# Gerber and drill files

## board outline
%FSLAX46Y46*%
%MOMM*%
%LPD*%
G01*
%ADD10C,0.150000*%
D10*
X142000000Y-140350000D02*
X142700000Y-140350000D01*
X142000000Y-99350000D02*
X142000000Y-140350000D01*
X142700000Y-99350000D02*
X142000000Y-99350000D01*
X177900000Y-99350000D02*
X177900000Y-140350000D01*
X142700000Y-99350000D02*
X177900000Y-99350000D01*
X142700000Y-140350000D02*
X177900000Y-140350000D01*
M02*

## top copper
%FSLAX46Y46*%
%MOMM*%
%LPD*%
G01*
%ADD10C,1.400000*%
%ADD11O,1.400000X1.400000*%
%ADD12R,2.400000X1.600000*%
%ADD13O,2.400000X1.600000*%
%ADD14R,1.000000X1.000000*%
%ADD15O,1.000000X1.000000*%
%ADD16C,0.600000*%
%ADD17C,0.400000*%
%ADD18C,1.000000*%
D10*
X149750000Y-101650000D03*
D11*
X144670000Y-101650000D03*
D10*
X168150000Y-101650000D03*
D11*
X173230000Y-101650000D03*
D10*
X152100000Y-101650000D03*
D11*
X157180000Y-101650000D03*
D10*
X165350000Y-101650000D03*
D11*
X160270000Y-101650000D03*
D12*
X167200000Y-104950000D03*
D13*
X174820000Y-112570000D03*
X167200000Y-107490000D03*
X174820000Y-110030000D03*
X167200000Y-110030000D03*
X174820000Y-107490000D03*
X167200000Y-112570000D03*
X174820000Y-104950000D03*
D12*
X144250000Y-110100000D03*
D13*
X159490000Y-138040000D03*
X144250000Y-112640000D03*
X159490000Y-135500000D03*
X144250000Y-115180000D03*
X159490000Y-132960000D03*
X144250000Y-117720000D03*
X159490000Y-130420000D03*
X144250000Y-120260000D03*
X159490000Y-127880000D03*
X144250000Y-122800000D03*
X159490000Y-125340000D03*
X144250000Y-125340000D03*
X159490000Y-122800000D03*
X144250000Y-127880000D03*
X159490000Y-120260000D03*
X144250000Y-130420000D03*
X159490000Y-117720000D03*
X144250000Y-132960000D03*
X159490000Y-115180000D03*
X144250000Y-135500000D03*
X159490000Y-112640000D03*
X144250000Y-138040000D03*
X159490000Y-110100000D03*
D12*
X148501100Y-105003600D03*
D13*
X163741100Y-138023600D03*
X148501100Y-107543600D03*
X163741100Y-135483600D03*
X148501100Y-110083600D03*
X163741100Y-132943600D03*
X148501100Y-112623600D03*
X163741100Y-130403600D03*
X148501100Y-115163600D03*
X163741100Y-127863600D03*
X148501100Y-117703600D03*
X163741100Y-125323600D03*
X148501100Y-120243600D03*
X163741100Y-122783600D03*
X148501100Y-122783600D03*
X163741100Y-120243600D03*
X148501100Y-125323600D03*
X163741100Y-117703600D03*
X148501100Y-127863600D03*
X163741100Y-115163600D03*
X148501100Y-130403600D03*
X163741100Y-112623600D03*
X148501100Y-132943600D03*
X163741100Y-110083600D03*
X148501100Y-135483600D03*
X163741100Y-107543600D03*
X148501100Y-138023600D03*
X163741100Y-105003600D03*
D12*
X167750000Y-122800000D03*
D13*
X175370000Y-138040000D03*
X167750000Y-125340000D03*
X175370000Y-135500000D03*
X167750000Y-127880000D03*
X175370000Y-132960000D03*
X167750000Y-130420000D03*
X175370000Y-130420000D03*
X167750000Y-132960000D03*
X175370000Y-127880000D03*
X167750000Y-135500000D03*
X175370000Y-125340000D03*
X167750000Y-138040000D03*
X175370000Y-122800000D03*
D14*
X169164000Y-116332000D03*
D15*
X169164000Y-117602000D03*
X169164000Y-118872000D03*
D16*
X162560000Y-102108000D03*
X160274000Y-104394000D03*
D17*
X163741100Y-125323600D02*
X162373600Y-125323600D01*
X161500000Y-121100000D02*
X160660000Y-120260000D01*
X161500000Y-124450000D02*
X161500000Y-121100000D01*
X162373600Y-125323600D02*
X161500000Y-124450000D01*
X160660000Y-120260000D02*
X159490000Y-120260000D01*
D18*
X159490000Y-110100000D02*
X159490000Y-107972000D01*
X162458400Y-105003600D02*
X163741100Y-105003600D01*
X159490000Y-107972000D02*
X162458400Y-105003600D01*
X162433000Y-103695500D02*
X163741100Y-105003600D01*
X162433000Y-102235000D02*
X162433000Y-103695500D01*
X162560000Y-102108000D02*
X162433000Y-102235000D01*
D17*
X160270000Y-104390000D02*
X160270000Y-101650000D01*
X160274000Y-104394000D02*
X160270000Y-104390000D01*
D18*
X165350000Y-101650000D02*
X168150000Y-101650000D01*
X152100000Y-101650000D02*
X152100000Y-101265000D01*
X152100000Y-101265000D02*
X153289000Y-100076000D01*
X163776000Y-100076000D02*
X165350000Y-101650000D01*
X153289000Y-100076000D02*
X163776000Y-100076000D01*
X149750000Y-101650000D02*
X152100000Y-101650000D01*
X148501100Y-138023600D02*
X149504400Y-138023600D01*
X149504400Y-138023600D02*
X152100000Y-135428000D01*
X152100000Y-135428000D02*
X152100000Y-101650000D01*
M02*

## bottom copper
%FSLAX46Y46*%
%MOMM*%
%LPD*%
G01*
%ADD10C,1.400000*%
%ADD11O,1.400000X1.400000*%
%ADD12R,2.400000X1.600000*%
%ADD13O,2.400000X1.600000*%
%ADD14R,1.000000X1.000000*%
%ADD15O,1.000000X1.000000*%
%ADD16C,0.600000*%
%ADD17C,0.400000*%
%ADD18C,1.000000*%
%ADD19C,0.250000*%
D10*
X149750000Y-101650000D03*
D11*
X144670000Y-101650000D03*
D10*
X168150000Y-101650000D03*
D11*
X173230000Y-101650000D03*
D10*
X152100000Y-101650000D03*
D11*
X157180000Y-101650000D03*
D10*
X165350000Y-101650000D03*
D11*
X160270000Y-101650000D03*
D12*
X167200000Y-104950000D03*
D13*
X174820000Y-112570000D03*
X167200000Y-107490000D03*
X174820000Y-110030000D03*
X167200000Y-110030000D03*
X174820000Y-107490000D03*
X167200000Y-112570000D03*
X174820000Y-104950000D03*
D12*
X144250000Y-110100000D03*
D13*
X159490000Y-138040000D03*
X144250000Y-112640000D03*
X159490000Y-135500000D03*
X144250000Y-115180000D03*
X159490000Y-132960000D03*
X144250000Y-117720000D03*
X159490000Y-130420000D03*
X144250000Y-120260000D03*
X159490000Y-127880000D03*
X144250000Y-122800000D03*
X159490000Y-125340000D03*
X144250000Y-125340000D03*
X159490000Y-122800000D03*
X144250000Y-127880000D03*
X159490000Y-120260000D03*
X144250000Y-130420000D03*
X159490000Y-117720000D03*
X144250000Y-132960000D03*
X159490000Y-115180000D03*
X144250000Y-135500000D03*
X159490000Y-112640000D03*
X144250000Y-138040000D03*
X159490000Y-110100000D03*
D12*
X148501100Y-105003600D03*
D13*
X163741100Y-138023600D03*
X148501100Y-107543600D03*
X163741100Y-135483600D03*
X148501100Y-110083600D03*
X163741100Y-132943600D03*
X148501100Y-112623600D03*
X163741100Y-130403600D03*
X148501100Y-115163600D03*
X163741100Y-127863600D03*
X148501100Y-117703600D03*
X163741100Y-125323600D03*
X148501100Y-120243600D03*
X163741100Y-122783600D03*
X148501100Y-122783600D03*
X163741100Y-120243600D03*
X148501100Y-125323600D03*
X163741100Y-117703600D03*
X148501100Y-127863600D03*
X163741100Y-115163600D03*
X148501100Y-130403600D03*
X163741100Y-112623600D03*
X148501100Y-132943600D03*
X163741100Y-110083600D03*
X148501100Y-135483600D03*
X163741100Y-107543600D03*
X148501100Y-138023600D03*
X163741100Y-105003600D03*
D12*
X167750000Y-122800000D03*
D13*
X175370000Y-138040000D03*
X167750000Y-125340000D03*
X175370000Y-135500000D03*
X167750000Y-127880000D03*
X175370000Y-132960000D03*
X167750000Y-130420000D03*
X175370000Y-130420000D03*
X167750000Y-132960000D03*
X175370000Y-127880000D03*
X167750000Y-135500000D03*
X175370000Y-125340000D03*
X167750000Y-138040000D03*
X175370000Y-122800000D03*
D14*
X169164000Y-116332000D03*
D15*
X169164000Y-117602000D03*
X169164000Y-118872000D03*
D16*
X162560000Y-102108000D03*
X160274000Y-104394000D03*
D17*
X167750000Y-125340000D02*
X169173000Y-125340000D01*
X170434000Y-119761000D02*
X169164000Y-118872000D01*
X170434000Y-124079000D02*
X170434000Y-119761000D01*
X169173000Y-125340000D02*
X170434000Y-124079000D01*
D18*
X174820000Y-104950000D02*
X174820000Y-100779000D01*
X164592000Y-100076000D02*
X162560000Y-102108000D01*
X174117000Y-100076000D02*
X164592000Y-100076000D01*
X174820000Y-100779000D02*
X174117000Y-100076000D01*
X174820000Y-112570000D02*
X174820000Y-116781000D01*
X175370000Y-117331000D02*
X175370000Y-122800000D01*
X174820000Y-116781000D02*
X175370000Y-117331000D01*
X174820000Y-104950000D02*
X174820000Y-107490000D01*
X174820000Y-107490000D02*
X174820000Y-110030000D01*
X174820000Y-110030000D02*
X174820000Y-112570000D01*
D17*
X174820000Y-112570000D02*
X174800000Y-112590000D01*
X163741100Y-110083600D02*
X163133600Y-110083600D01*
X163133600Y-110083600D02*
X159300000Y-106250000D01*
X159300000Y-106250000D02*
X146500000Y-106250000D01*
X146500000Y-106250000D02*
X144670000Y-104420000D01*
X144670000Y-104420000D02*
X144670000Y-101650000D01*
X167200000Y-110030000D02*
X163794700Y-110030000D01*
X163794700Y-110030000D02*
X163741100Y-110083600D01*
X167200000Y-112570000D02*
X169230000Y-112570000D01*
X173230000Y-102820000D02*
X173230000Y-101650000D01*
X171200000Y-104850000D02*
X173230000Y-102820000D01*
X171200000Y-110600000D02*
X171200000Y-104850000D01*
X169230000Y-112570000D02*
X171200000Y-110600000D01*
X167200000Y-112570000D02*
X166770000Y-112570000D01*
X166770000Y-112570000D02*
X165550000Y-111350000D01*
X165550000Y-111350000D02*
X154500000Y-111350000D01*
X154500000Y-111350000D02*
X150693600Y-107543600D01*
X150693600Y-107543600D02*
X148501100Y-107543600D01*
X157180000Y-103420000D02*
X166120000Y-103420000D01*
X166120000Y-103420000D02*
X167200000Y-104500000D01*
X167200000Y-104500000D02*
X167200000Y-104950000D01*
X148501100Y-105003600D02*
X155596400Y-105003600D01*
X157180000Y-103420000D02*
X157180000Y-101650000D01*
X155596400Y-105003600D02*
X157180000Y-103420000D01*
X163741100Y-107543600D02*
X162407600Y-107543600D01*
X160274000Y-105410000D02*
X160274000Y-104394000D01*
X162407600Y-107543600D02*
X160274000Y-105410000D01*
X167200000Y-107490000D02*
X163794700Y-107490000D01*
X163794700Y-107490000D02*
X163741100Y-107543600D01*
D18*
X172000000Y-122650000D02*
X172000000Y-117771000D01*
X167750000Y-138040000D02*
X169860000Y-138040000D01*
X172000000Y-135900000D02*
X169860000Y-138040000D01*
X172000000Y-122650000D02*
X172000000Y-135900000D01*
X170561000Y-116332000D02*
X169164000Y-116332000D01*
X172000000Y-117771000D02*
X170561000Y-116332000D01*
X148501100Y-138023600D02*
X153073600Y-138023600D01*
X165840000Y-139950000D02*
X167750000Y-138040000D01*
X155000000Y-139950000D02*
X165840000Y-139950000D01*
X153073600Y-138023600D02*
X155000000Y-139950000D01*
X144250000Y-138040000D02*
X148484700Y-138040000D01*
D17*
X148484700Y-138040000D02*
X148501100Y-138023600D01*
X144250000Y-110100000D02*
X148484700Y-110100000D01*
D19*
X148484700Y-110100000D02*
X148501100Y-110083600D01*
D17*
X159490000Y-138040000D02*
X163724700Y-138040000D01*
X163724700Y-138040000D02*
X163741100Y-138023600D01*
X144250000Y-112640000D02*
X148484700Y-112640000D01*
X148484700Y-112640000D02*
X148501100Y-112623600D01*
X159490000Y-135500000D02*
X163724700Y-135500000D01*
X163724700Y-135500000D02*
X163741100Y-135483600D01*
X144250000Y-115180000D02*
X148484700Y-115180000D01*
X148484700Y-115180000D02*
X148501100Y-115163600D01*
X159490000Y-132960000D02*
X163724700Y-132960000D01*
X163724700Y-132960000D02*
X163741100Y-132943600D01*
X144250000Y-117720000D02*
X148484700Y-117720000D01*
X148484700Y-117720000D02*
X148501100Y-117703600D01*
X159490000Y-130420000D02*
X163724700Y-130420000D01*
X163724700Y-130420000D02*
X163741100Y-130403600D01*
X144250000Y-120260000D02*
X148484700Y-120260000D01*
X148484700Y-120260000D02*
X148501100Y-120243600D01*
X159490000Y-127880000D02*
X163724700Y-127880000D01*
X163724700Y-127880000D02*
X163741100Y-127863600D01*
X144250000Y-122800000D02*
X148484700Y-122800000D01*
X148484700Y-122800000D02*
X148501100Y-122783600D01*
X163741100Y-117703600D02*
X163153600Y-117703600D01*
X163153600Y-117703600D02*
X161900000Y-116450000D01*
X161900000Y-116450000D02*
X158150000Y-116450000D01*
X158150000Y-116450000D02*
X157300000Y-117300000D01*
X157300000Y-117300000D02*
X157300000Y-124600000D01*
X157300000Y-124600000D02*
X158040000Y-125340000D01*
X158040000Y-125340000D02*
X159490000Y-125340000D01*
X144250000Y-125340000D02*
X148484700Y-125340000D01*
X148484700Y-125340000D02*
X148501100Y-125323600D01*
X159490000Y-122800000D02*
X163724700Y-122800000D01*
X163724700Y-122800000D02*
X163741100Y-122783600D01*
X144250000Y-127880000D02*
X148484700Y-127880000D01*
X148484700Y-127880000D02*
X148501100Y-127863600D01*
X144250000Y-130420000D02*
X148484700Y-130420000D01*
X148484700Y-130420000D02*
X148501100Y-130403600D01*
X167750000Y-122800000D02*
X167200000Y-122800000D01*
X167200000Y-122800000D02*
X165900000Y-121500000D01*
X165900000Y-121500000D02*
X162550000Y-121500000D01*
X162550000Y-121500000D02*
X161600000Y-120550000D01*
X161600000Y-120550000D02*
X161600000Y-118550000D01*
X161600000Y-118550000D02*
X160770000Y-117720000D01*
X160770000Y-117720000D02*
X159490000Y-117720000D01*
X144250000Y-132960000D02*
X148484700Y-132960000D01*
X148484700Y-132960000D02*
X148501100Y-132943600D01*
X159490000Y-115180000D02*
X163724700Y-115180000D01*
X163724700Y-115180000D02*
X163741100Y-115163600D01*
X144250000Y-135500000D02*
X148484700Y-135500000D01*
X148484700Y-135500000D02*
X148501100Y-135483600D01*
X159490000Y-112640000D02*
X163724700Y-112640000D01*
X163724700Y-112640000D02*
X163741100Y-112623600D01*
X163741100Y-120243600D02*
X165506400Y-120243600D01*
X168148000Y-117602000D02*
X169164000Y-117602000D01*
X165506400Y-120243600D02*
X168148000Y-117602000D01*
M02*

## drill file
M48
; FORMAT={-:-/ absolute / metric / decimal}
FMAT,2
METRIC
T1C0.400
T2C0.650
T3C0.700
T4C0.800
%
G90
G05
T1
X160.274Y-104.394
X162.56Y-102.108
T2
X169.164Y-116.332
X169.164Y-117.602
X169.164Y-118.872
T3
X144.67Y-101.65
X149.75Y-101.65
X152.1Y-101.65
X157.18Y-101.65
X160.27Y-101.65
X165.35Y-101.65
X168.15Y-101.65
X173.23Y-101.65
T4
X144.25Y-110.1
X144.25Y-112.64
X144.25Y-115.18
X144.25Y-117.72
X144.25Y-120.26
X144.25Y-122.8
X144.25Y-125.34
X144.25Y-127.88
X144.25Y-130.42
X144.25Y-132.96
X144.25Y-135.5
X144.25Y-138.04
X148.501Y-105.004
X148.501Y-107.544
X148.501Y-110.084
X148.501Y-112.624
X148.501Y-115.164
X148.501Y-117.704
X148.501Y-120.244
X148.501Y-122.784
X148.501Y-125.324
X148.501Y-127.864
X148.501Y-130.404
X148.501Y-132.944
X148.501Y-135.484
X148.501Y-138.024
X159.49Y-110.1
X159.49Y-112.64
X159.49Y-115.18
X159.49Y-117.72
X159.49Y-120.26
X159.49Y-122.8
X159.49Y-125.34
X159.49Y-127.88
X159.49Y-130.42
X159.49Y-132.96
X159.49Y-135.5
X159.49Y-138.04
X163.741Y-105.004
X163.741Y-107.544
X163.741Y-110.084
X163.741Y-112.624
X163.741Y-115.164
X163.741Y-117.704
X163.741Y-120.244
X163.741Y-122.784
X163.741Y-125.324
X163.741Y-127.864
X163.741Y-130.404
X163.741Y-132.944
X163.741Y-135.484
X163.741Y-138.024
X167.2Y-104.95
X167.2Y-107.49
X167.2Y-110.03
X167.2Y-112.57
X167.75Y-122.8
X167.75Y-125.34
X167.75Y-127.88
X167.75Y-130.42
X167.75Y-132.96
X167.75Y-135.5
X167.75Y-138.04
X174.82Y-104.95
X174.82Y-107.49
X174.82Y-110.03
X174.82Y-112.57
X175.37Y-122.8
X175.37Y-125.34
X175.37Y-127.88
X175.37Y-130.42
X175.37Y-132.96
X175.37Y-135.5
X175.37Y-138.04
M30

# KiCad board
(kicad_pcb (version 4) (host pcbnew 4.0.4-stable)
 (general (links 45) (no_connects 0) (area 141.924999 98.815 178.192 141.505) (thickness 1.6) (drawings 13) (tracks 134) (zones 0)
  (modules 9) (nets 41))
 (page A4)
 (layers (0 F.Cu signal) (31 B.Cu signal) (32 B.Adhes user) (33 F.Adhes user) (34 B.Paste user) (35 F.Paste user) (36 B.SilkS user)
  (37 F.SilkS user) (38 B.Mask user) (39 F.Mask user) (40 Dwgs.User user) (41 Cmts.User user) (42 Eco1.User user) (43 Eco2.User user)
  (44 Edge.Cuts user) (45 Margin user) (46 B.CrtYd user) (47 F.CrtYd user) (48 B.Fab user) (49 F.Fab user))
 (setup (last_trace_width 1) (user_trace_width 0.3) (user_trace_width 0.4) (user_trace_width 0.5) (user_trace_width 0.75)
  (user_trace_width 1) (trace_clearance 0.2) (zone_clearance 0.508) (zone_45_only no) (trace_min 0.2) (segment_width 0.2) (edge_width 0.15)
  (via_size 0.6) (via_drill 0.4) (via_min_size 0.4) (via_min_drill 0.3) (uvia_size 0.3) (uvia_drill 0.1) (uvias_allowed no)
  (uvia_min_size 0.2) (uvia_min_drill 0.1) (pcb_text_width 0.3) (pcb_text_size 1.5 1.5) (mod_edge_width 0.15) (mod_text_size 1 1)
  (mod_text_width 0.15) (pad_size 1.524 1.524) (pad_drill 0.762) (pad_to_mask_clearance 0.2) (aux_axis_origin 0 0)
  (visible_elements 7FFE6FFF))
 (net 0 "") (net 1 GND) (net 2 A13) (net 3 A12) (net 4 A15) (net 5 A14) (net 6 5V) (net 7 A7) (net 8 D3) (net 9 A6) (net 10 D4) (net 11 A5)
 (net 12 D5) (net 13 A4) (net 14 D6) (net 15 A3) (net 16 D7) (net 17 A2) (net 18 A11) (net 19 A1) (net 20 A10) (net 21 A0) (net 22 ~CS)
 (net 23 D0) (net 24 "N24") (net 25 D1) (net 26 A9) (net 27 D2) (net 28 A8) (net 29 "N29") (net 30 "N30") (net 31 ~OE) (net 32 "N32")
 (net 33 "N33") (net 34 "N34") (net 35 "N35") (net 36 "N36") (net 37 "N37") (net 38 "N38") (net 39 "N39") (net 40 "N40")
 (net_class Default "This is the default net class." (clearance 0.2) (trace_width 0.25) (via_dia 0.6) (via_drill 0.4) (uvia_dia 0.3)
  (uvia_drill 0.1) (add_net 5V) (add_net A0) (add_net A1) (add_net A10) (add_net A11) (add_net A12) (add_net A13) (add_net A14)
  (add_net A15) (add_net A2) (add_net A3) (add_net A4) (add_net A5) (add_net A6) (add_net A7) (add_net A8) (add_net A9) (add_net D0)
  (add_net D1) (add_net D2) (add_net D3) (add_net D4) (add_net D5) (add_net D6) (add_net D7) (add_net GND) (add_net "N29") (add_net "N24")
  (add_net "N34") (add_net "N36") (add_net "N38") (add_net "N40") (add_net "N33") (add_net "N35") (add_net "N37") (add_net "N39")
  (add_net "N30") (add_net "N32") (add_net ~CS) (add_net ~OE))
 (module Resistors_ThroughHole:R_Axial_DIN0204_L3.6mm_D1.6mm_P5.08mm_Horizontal (layer F.Cu) (at 149.75 101.65 180)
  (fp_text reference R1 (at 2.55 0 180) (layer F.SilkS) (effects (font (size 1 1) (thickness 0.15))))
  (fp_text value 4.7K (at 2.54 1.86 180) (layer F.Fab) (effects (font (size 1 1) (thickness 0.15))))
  (pad 1 thru_hole circle (at 0 0 180) (size 1.4 1.4) (drill 0.7) (layers *.Cu *.Mask) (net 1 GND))
  (pad 2 thru_hole oval (at 5.08 0 180) (size 1.4 1.4) (drill 0.7) (layers *.Cu *.Mask) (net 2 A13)))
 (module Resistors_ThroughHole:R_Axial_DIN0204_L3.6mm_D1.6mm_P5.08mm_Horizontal (layer F.Cu) (at 168.15 101.65)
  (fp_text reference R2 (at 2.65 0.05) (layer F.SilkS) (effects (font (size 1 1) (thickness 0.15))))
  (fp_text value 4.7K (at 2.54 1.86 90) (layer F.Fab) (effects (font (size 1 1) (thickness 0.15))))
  (pad 1 thru_hole circle (at 0 0) (size 1.4 1.4) (drill 0.7) (layers *.Cu *.Mask) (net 1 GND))
  (pad 2 thru_hole oval (at 5.08 0) (size 1.4 1.4) (drill 0.7) (layers *.Cu *.Mask) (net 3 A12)))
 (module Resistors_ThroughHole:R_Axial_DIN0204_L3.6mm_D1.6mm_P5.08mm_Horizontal (layer F.Cu) (at 152.1 101.65)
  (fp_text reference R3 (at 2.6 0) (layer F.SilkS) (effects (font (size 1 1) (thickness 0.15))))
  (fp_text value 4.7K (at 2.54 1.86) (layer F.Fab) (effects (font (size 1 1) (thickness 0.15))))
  (pad 1 thru_hole circle (at 0 0) (size 1.4 1.4) (drill 0.7) (layers *.Cu *.Mask) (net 1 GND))
  (pad 2 thru_hole oval (at 5.08 0) (size 1.4 1.4) (drill 0.7) (layers *.Cu *.Mask) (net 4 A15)))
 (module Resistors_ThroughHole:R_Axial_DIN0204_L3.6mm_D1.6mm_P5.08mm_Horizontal (layer F.Cu) (at 165.35 101.65 180)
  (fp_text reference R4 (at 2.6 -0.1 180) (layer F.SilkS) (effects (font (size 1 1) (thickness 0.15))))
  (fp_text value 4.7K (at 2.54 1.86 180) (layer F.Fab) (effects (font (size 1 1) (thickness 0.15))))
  (pad 1 thru_hole circle (at 0 0 180) (size 1.4 1.4) (drill 0.7) (layers *.Cu *.Mask) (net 1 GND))
  (pad 2 thru_hole oval (at 5.08 0 180) (size 1.4 1.4) (drill 0.7) (layers *.Cu *.Mask) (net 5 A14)))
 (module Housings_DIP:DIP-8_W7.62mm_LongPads (layer F.Cu) (at 167.2 104.95)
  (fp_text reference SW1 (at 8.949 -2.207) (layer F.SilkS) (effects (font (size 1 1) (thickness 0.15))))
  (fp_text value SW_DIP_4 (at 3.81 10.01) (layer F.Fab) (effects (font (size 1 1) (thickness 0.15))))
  (pad 1 thru_hole rect (at 0 0) (size 2.4 1.6) (drill 0.8) (layers *.Cu *.Mask) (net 4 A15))
  (pad 5 thru_hole oval (at 7.62 7.62) (size 2.4 1.6) (drill 0.8) (layers *.Cu *.Mask) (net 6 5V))
  (pad 2 thru_hole oval (at 0 2.54) (size 2.4 1.6) (drill 0.8) (layers *.Cu *.Mask) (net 5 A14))
  (pad 6 thru_hole oval (at 7.62 5.08) (size 2.4 1.6) (drill 0.8) (layers *.Cu *.Mask) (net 6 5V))
  (pad 3 thru_hole oval (at 0 5.08) (size 2.4 1.6) (drill 0.8) (layers *.Cu *.Mask) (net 2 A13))
  (pad 7 thru_hole oval (at 7.62 2.54) (size 2.4 1.6) (drill 0.8) (layers *.Cu *.Mask) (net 6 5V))
  (pad 4 thru_hole oval (at 0 7.62) (size 2.4 1.6) (drill 0.8) (layers *.Cu *.Mask) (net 3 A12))
  (pad 8 thru_hole oval (at 7.62 0) (size 2.4 1.6) (drill 0.8) (layers *.Cu *.Mask) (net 6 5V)))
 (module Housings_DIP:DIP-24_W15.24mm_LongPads (layer F.Cu) (at 144.25 110.1)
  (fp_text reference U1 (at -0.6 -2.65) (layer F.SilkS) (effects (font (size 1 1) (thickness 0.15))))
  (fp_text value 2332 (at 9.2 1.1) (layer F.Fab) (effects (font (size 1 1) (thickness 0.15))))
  (pad 1 thru_hole rect (at 0 0) (size 2.4 1.6) (drill 0.8) (layers *.Cu *.Mask) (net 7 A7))
  (pad 13 thru_hole oval (at 15.24 27.94) (size 2.4 1.6) (drill 0.8) (layers *.Cu *.Mask) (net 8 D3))
  (pad 2 thru_hole oval (at 0 2.54) (size 2.4 1.6) (drill 0.8) (layers *.Cu *.Mask) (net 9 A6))
  (pad 14 thru_hole oval (at 15.24 25.4) (size 2.4 1.6) (drill 0.8) (layers *.Cu *.Mask) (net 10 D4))
  (pad 3 thru_hole oval (at 0 5.08) (size 2.4 1.6) (drill 0.8) (layers *.Cu *.Mask) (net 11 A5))
  (pad 15 thru_hole oval (at 15.24 22.86) (size 2.4 1.6) (drill 0.8) (layers *.Cu *.Mask) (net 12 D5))
  (pad 4 thru_hole oval (at 0 7.62) (size 2.4 1.6) (drill 0.8) (layers *.Cu *.Mask) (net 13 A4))
  (pad 16 thru_hole oval (at 15.24 20.32) (size 2.4 1.6) (drill 0.8) (layers *.Cu *.Mask) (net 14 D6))
  (pad 5 thru_hole oval (at 0 10.16) (size 2.4 1.6) (drill 0.8) (layers *.Cu *.Mask) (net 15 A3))
  (pad 17 thru_hole oval (at 15.24 17.78) (size 2.4 1.6) (drill 0.8) (layers *.Cu *.Mask) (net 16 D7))
  (pad 6 thru_hole oval (at 0 12.7) (size 2.4 1.6) (drill 0.8) (layers *.Cu *.Mask) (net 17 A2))
  (pad 18 thru_hole oval (at 15.24 15.24) (size 2.4 1.6) (drill 0.8) (layers *.Cu *.Mask) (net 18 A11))
  (pad 7 thru_hole oval (at 0 15.24) (size 2.4 1.6) (drill 0.8) (layers *.Cu *.Mask) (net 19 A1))
  (pad 19 thru_hole oval (at 15.24 12.7) (size 2.4 1.6) (drill 0.8) (layers *.Cu *.Mask) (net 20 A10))
  (pad 8 thru_hole oval (at 0 17.78) (size 2.4 1.6) (drill 0.8) (layers *.Cu *.Mask) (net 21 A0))
  (pad 20 thru_hole oval (at 15.24 10.16) (size 2.4 1.6) (drill 0.8) (layers *.Cu *.Mask) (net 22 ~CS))
  (pad 9 thru_hole oval (at 0 20.32) (size 2.4 1.6) (drill 0.8) (layers *.Cu *.Mask) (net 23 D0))
  (pad 21 thru_hole oval (at 15.24 7.62) (size 2.4 1.6) (drill 0.8) (layers *.Cu *.Mask) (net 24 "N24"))
  (pad 10 thru_hole oval (at 0 22.86) (size 2.4 1.6) (drill 0.8) (layers *.Cu *.Mask) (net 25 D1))
  (pad 22 thru_hole oval (at 15.24 5.08) (size 2.4 1.6) (drill 0.8) (layers *.Cu *.Mask) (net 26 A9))
  (pad 11 thru_hole oval (at 0 25.4) (size 2.4 1.6) (drill 0.8) (layers *.Cu *.Mask) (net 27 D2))
  (pad 23 thru_hole oval (at 15.24 2.54) (size 2.4 1.6) (drill 0.8) (layers *.Cu *.Mask) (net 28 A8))
  (pad 12 thru_hole oval (at 0 27.94) (size 2.4 1.6) (drill 0.8) (layers *.Cu *.Mask) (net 1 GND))
  (pad 24 thru_hole oval (at 15.24 0) (size 2.4 1.6) (drill 0.8) (layers *.Cu *.Mask) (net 6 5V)))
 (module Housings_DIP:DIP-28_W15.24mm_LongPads (layer F.Cu) (at 148.5011 105.0036)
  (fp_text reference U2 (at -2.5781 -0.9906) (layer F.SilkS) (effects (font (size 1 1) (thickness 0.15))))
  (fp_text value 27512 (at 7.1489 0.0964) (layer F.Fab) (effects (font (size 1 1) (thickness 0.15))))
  (pad 1 thru_hole rect (at 0 0) (size 2.4 1.6) (drill 0.8) (layers *.Cu *.Mask) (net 4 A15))
  (pad 15 thru_hole oval (at 15.24 33.02) (size 2.4 1.6) (drill 0.8) (layers *.Cu *.Mask) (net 8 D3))
  (pad 2 thru_hole oval (at 0 2.54) (size 2.4 1.6) (drill 0.8) (layers *.Cu *.Mask) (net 3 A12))
  (pad 16 thru_hole oval (at 15.24 30.48) (size 2.4 1.6) (drill 0.8) (layers *.Cu *.Mask) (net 10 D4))
  (pad 3 thru_hole oval (at 0 5.08) (size 2.4 1.6) (drill 0.8) (layers *.Cu *.Mask) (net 7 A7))
  (pad 17 thru_hole oval (at 15.24 27.94) (size 2.4 1.6) (drill 0.8) (layers *.Cu *.Mask) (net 12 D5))
  (pad 4 thru_hole oval (at 0 7.62) (size 2.4 1.6) (drill 0.8) (layers *.Cu *.Mask) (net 9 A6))
  (pad 18 thru_hole oval (at 15.24 25.4) (size 2.4 1.6) (drill 0.8) (layers *.Cu *.Mask) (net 14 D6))
  (pad 5 thru_hole oval (at 0 10.16) (size 2.4 1.6) (drill 0.8) (layers *.Cu *.Mask) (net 11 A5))
  (pad 19 thru_hole oval (at 15.24 22.86) (size 2.4 1.6) (drill 0.8) (layers *.Cu *.Mask) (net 16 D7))
  (pad 6 thru_hole oval (at 0 12.7) (size 2.4 1.6) (drill 0.8) (layers *.Cu *.Mask) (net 13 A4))
  (pad 20 thru_hole oval (at 15.24 20.32) (size 2.4 1.6) (drill 0.8) (layers *.Cu *.Mask) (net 22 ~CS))
  (pad 7 thru_hole oval (at 0 15.24) (size 2.4 1.6) (drill 0.8) (layers *.Cu *.Mask) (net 15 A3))
  (pad 21 thru_hole oval (at 15.24 17.78) (size 2.4 1.6) (drill 0.8) (layers *.Cu *.Mask) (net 20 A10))
  (pad 8 thru_hole oval (at 0 17.78) (size 2.4 1.6) (drill 0.8) (layers *.Cu *.Mask) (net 17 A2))
  (pad 22 thru_hole oval (at 15.24 15.24) (size 2.4 1.6) (drill 0.8) (layers *.Cu *.Mask) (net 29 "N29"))
  (pad 9 thru_hole oval (at 0 20.32) (size 2.4 1.6) (drill 0.8) (layers *.Cu *.Mask) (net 19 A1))
  (pad 23 thru_hole oval (at 15.24 12.7) (size 2.4 1.6) (drill 0.8) (layers *.Cu *.Mask) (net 18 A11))
  (pad 10 thru_hole oval (at 0 22.86) (size 2.4 1.6) (drill 0.8) (layers *.Cu *.Mask) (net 21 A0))
  (pad 24 thru_hole oval (at 15.24 10.16) (size 2.4 1.6) (drill 0.8) (layers *.Cu *.Mask) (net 26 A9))
  (pad 11 thru_hole oval (at 0 25.4) (size 2.4 1.6) (drill 0.8) (layers *.Cu *.Mask) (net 23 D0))
  (pad 25 thru_hole oval (at 15.24 7.62) (size 2.4 1.6) (drill 0.8) (layers *.Cu *.Mask) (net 28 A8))
  (pad 12 thru_hole oval (at 0 27.94) (size 2.4 1.6) (drill 0.8) (layers *.Cu *.Mask) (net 25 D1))
  (pad 26 thru_hole oval (at 15.24 5.08) (size 2.4 1.6) (drill 0.8) (layers *.Cu *.Mask) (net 2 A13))
  (pad 13 thru_hole oval (at 0 30.48) (size 2.4 1.6) (drill 0.8) (layers *.Cu *.Mask) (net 27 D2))
  (pad 27 thru_hole oval (at 15.24 2.54) (size 2.4 1.6) (drill 0.8) (layers *.Cu *.Mask) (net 5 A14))
  (pad 14 thru_hole oval (at 0 33.02) (size 2.4 1.6) (drill 0.8) (layers *.Cu *.Mask) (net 1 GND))
  (pad 28 thru_hole oval (at 15.24 0) (size 2.4 1.6) (drill 0.8) (layers *.Cu *.Mask) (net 6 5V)))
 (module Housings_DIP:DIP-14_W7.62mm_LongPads (layer F.Cu) (at 167.75 122.8)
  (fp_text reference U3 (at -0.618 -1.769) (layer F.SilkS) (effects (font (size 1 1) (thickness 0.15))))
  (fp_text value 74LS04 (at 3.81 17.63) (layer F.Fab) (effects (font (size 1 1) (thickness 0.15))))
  (pad 1 thru_hole rect (at 0 0) (size 2.4 1.6) (drill 0.8) (layers *.Cu *.Mask) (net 24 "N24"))
  (pad 8 thru_hole oval (at 7.62 15.24) (size 2.4 1.6) (drill 0.8) (layers *.Cu *.Mask) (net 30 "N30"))
  (pad 2 thru_hole oval (at 0 2.54) (size 2.4 1.6) (drill 0.8) (layers *.Cu *.Mask) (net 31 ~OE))
  (pad 9 thru_hole oval (at 7.62 12.7) (size 2.4 1.6) (drill 0.8) (layers *.Cu *.Mask) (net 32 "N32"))
  (pad 3 thru_hole oval (at 0 5.08) (size 2.4 1.6) (drill 0.8) (layers *.Cu *.Mask) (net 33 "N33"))
  (pad 10 thru_hole oval (at 7.62 10.16) (size 2.4 1.6) (drill 0.8) (layers *.Cu *.Mask) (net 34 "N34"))
  (pad 4 thru_hole oval (at 0 7.62) (size 2.4 1.6) (drill 0.8) (layers *.Cu *.Mask) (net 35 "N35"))
  (pad 11 thru_hole oval (at 7.62 7.62) (size 2.4 1.6) (drill 0.8) (layers *.Cu *.Mask) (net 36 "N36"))
  (pad 5 thru_hole oval (at 0 10.16) (size 2.4 1.6) (drill 0.8) (layers *.Cu *.Mask) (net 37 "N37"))
  (pad 12 thru_hole oval (at 7.62 5.08) (size 2.4 1.6) (drill 0.8) (layers *.Cu *.Mask) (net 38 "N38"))
  (pad 6 thru_hole oval (at 0 12.7) (size 2.4 1.6) (drill 0.8) (layers *.Cu *.Mask) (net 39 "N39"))
  (pad 13 thru_hole oval (at 7.62 2.54) (size 2.4 1.6) (drill 0.8) (layers *.Cu *.Mask) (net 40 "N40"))
  (pad 7 thru_hole oval (at 0 15.24) (size 2.4 1.6) (drill 0.8) (layers *.Cu *.Mask) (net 1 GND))
  (pad 14 thru_hole oval (at 7.62 0) (size 2.4 1.6) (drill 0.8) (layers *.Cu *.Mask) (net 6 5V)))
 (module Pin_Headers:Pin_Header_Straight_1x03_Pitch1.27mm (layer F.Cu) (at 169.164 116.332)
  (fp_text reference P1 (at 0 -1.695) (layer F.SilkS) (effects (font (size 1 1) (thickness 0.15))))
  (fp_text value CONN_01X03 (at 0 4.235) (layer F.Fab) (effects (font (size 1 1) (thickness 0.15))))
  (pad 1 thru_hole rect (at 0 0) (size 1 1) (drill 0.65) (layers *.Cu *.Mask) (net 1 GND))
  (pad 2 thru_hole oval (at 0 1.27) (size 1 1) (drill 0.65) (layers *.Cu *.Mask) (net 29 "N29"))
  (pad 3 thru_hole oval (at 0 2.54) (size 1 1) (drill 0.65) (layers *.Cu *.Mask) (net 31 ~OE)))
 (gr_line (start 142 140.35) (end 142.7 140.35) (angle 90) (layer Edge.Cuts) (width 0.15))
 (gr_line (start 142 99.35) (end 142 140.35) (angle 90) (layer Edge.Cuts) (width 0.15))
 (gr_line (start 142.7 99.35) (end 142 99.35) (angle 90) (layer Edge.Cuts) (width 0.15))
 (gr_line (start 177.9 99.35) (end 177.9 140.35) (angle 90) (layer Edge.Cuts) (width 0.15))
 (gr_line (start 142.7 99.35) (end 177.9 99.35) (angle 90) (layer Edge.Cuts) (width 0.15))
 (gr_line (start 142.7 140.35) (end 177.9 140.35) (angle 90) (layer Edge.Cuts) (width 0.15))
 (segment (start 167.75 125.34) (end 169.173 125.34) (width 0.4) (layer B.Cu) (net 31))
 (segment (start 170.434 119.761) (end 169.164 118.872) (width 0.4) (layer B.Cu) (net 31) (status 20))
 (segment (start 170.434 124.079) (end 170.434 119.761) (width 0.4) (layer B.Cu) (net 31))
 (segment (start 169.173 125.34) (end 170.434 124.079) (width 0.4) (layer B.Cu) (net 31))
 (segment (start 163.7411 125.3236) (end 162.3736 125.3236) (width 0.4) (layer F.Cu) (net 22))
 (segment (start 161.5 121.1) (end 160.66 120.26) (width 0.4) (layer F.Cu) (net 22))
 (segment (start 161.5 124.45) (end 161.5 121.1) (width 0.4) (layer F.Cu) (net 22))
 (segment (start 162.3736 125.3236) (end 161.5 124.45) (width 0.4) (layer F.Cu) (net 22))
 (segment (start 160.66 120.26) (end 159.49 120.26) (width 0.4) (layer F.Cu) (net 22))
 (segment (start 159.49 110.1) (end 159.49 107.972) (width 1) (layer F.Cu) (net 6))
 (segment (start 162.4584 105.0036) (end 163.7411 105.0036) (width 1) (layer F.Cu) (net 6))
 (segment (start 159.49 107.972) (end 162.4584 105.0036) (width 1) (layer F.Cu) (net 6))
 (segment (start 174.82 104.95) (end 174.82 100.779) (width 1) (layer B.Cu) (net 6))
 (segment (start 162.433 103.6955) (end 163.7411 105.0036) (width 1) (layer F.Cu) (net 6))
 (segment (start 162.433 102.235) (end 162.433 103.6955) (width 1) (layer F.Cu) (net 6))
 (segment (start 162.56 102.108) (end 162.433 102.235) (width 1) (layer F.Cu) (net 6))
 (via (at 162.56 102.108) (size 0.6) (drill 0.4) (layers F.Cu B.Cu) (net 6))
 (segment (start 164.592 100.076) (end 162.56 102.108) (width 1) (layer B.Cu) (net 6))
 (segment (start 174.117 100.076) (end 164.592 100.076) (width 1) (layer B.Cu) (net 6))
 (segment (start 174.82 100.779) (end 174.117 100.076) (width 1) (layer B.Cu) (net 6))
 (segment (start 174.82 112.57) (end 174.82 116.781) (width 1) (layer B.Cu) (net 6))
 (segment (start 175.37 117.331) (end 175.37 122.8) (width 1) (layer B.Cu) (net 6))
 (segment (start 174.82 116.781) (end 175.37 117.331) (width 1) (layer B.Cu) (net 6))
 (segment (start 174.82 104.95) (end 174.82 107.49) (width 1) (layer B.Cu) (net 6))
 (segment (start 174.82 107.49) (end 174.82 110.03) (width 1) (layer B.Cu) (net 6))
 (segment (start 174.82 110.03) (end 174.82 112.57) (width 1) (layer B.Cu) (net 6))
 (segment (start 174.82 112.57) (end 174.8 112.59) (width 0.4) (layer B.Cu) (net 6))
 (segment (start 163.7411 110.0836) (end 163.1336 110.0836) (width 0.4) (layer B.Cu) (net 2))
 (segment (start 163.1336 110.0836) (end 159.3 106.25) (width 0.4) (layer B.Cu) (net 2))
 (segment (start 159.3 106.25) (end 146.5 106.25) (width 0.4) (layer B.Cu) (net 2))
 (segment (start 146.5 106.25) (end 144.67 104.42) (width 0.4) (layer B.Cu) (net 2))
 (segment (start 144.67 104.42) (end 144.67 101.65) (width 0.4) (layer B.Cu) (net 2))
 (segment (start 167.2 110.03) (end 163.7947 110.03) (width 0.4) (layer B.Cu) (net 2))
 (segment (start 163.7947 110.03) (end 163.7411 110.0836) (width 0.4) (layer B.Cu) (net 2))
 (segment (start 167.2 112.57) (end 169.23 112.57) (width 0.4) (layer B.Cu) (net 3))
 (segment (start 173.23 102.82) (end 173.23 101.65) (width 0.4) (layer B.Cu) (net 3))
 (segment (start 171.2 104.85) (end 173.23 102.82) (width 0.4) (layer B.Cu) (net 3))
 (segment (start 171.2 110.6) (end 171.2 104.85) (width 0.4) (layer B.Cu) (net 3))
 (segment (start 169.23 112.57) (end 171.2 110.6) (width 0.4) (layer B.Cu) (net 3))
 (segment (start 167.2 112.57) (end 166.77 112.57) (width 0.4) (layer B.Cu) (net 3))
 (segment (start 166.77 112.57) (end 165.55 111.35) (width 0.4) (layer B.Cu) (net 3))
 (segment (start 165.55 111.35) (end 154.5 111.35) (width 0.4) (layer B.Cu) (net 3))
 (segment (start 154.5 111.35) (end 150.6936 107.5436) (width 0.4) (layer B.Cu) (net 3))
 (segment (start 150.6936 107.5436) (end 148.5011 107.5436) (width 0.4) (layer B.Cu) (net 3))
 (segment (start 157.18 103.42) (end 166.12 103.42) (width 0.4) (layer B.Cu) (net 4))
 (segment (start 166.12 103.42) (end 167.2 104.5) (width 0.4) (layer B.Cu) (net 4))
 (segment (start 167.2 104.5) (end 167.2 104.95) (width 0.4) (layer B.Cu) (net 4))
 (segment (start 148.5011 105.0036) (end 155.5964 105.0036) (width 0.4) (layer B.Cu) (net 4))
 (segment (start 157.18 103.42) (end 157.18 101.65) (width 0.4) (layer B.Cu) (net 4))
 (segment (start 155.5964 105.0036) (end 157.18 103.42) (width 0.4) (layer B.Cu) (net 4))
 (segment (start 163.7411 107.5436) (end 162.4076 107.5436) (width 0.4) (layer B.Cu) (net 5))
 (segment (start 160.27 104.39) (end 160.27 101.65) (width 0.4) (layer F.Cu) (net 5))
 (segment (start 160.274 104.394) (end 160.27 104.39) (width 0.4) (layer F.Cu) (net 5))
 (via (at 160.274 104.394) (size 0.6) (drill 0.4) (layers F.Cu B.Cu) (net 5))
 (segment (start 160.274 105.41) (end 160.274 104.394) (width 0.4) (layer B.Cu) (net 5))
 (segment (start 162.4076 107.5436) (end 160.274 105.41) (width 0.4) (layer B.Cu) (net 5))
 (segment (start 167.2 107.49) (end 163.7947 107.49) (width 0.4) (layer B.Cu) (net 5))
 (segment (start 163.7947 107.49) (end 163.7411 107.5436) (width 0.4) (layer B.Cu) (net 5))
 (segment (start 165.35 101.65) (end 168.15 101.65) (width 1) (layer F.Cu) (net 1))
 (segment (start 152.1 101.65) (end 152.1 101.265) (width 1) (layer F.Cu) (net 1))
 (segment (start 152.1 101.265) (end 153.289 100.076) (width 1) (layer F.Cu) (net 1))
 (segment (start 163.776 100.076) (end 165.35 101.65) (width 1) (layer F.Cu) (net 1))
 (segment (start 153.289 100.076) (end 163.776 100.076) (width 1) (layer F.Cu) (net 1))
 (segment (start 149.75 101.65) (end 152.1 101.65) (width 1) (layer F.Cu) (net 1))
 (segment (start 148.5011 138.0236) (end 149.5044 138.0236) (width 1) (layer F.Cu) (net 1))
 (segment (start 149.5044 138.0236) (end 152.1 135.428) (width 1) (layer F.Cu) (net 1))
 (segment (start 152.1 135.428) (end 152.1 101.65) (width 1) (layer F.Cu) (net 1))
 (segment (start 172 122.65) (end 172 117.771) (width 1) (layer B.Cu) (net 1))
 (segment (start 167.75 138.04) (end 169.86 138.04) (width 1) (layer B.Cu) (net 1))
 (segment (start 172 135.9) (end 169.86 138.04) (width 1) (layer B.Cu) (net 1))
 (segment (start 172 122.65) (end 172 135.9) (width 1) (layer B.Cu) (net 1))
 (segment (start 170.561 116.332) (end 169.164 116.332) (width 1) (layer B.Cu) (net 1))
 (segment (start 172 117.771) (end 170.561 116.332) (width 1) (layer B.Cu) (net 1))
 (segment (start 148.5011 138.0236) (end 153.0736 138.0236) (width 1) (layer B.Cu) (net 1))
 (segment (start 165.84 139.95) (end 167.75 138.04) (width 1) (layer B.Cu) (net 1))
 (segment (start 155 139.95) (end 165.84 139.95) (width 1) (layer B.Cu) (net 1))
 (segment (start 153.0736 138.0236) (end 155 139.95) (width 1) (layer B.Cu) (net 1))
 (segment (start 144.25 138.04) (end 148.4847 138.04) (width 1) (layer B.Cu) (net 1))
 (segment (start 148.4847 138.04) (end 148.5011 138.0236) (width 0.4) (layer B.Cu) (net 1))
 (segment (start 144.25 110.1) (end 148.4847 110.1) (width 0.4) (layer B.Cu) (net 7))
 (segment (start 148.4847 110.1) (end 148.5011 110.0836) (width 0.25) (layer B.Cu) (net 7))
 (segment (start 159.49 138.04) (end 163.7247 138.04) (width 0.4) (layer B.Cu) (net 8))
 (segment (start 163.7247 138.04) (end 163.7411 138.0236) (width 0.4) (layer B.Cu) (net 8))
 (segment (start 144.25 112.64) (end 148.4847 112.64) (width 0.4) (layer B.Cu) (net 9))
 (segment (start 148.4847 112.64) (end 148.5011 112.6236) (width 0.4) (layer B.Cu) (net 9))
 (segment (start 159.49 135.5) (end 163.7247 135.5) (width 0.4) (layer B.Cu) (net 10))
 (segment (start 163.7247 135.5) (end 163.7411 135.4836) (width 0.4) (layer B.Cu) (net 10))
 (segment (start 144.25 115.18) (end 148.4847 115.18) (width 0.4) (layer B.Cu) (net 11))
 (segment (start 148.4847 115.18) (end 148.5011 115.1636) (width 0.4) (layer B.Cu) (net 11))
 (segment (start 159.49 132.96) (end 163.7247 132.96) (width 0.4) (layer B.Cu) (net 12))
 (segment (start 163.7247 132.96) (end 163.7411 132.9436) (width 0.4) (layer B.Cu) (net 12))
 (segment (start 144.25 117.72) (end 148.4847 117.72) (width 0.4) (layer B.Cu) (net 13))
 (segment (start 148.4847 117.72) (end 148.5011 117.7036) (width 0.4) (layer B.Cu) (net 13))
 (segment (start 159.49 130.42) (end 163.7247 130.42) (width 0.4) (layer B.Cu) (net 14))
 (segment (start 163.7247 130.42) (end 163.7411 130.4036) (width 0.4) (layer B.Cu) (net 14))
 (segment (start 144.25 120.26) (end 148.4847 120.26) (width 0.4) (layer B.Cu) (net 15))
 (segment (start 148.4847 120.26) (end 148.5011 120.2436) (width 0.4) (layer B.Cu) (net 15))
 (segment (start 159.49 127.88) (end 163.7247 127.88) (width 0.4) (layer B.Cu) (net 16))
 (segment (start 163.7247 127.88) (end 163.7411 127.8636) (width 0.4) (layer B.Cu) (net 16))
 (segment (start 144.25 122.8) (end 148.4847 122.8) (width 0.4) (layer B.Cu) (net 17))
 (segment (start 148.4847 122.8) (end 148.5011 122.7836) (width 0.4) (layer B.Cu) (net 17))
 (segment (start 163.7411 117.7036) (end 163.1536 117.7036) (width 0.4) (layer B.Cu) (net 18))
 (segment (start 163.1536 117.7036) (end 161.9 116.45) (width 0.4) (layer B.Cu) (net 18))
 (segment (start 161.9 116.45) (end 158.15 116.45) (width 0.4) (layer B.Cu) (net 18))
 (segment (start 158.15 116.45) (end 157.3 117.3) (width 0.4) (layer B.Cu) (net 18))
 (segment (start 157.3 117.3) (end 157.3 124.6) (width 0.4) (layer B.Cu) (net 18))
 (segment (start 157.3 124.6) (end 158.04 125.34) (width 0.4) (layer B.Cu) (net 18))
 (segment (start 158.04 125.34) (end 159.49 125.34) (width 0.4) (layer B.Cu) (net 18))
 (segment (start 144.25 125.34) (end 148.4847 125.34) (width 0.4) (layer B.Cu) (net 19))
 (segment (start 148.4847 125.34) (end 148.5011 125.3236) (width 0.4) (layer B.Cu) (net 19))
 (segment (start 159.49 122.8) (end 163.7247 122.8) (width 0.4) (layer B.Cu) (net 20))
 (segment (start 163.7247 122.8) (end 163.7411 122.7836) (width 0.4) (layer B.Cu) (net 20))
 (segment (start 144.25 127.88) (end 148.4847 127.88) (width 0.4) (layer B.Cu) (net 21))
 (segment (start 148.4847 127.88) (end 148.5011 127.8636) (width 0.4) (layer B.Cu) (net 21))
 (segment (start 144.25 130.42) (end 148.4847 130.42) (width 0.4) (layer B.Cu) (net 23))
 (segment (start 148.4847 130.42) (end 148.5011 130.4036) (width 0.4) (layer B.Cu) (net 23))
 (segment (start 167.75 122.8) (end 167.2 122.8) (width 0.4) (layer B.Cu) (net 24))
 (segment (start 167.2 122.8) (end 165.9 121.5) (width 0.4) (layer B.Cu) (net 24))
 (segment (start 165.9 121.5) (end 162.55 121.5) (width 0.4) (layer B.Cu) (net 24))
 (segment (start 162.55 121.5) (end 161.6 120.55) (width 0.4) (layer B.Cu) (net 24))
 (segment (start 161.6 120.55) (end 161.6 118.55) (width 0.4) (layer B.Cu) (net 24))
 (segment (start 161.6 118.55) (end 160.77 117.72) (width 0.4) (layer B.Cu) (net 24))
 (segment (start 160.77 117.72) (end 159.49 117.72) (width 0.4) (layer B.Cu) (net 24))
 (segment (start 144.25 132.96) (end 148.4847 132.96) (width 0.4) (layer B.Cu) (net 25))
 (segment (start 148.4847 132.96) (end 148.5011 132.9436) (width 0.4) (layer B.Cu) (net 25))
 (segment (start 159.49 115.18) (end 163.7247 115.18) (width 0.4) (layer B.Cu) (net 26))
 (segment (start 163.7247 115.18) (end 163.7411 115.1636) (width 0.4) (layer B.Cu) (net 26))
 (segment (start 144.25 135.5) (end 148.4847 135.5) (width 0.4) (layer B.Cu) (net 27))
 (segment (start 148.4847 135.5) (end 148.5011 135.4836) (width 0.4) (layer B.Cu) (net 27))
 (segment (start 159.49 112.64) (end 163.7247 112.64) (width 0.4) (layer B.Cu) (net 28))
 (segment (start 163.7247 112.64) (end 163.7411 112.6236) (width 0.4) (layer B.Cu) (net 28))
 (segment (start 163.7411 120.2436) (end 165.5064 120.2436) (width 0.4) (layer B.Cu) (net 29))
 (segment (start 168.148 117.602) (end 169.164 117.602) (width 0.4) (layer B.Cu) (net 29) (status 20))
 (segment (start 165.5064 120.2436) (end 168.148 117.602) (width 0.4) (layer B.Cu) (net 29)))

